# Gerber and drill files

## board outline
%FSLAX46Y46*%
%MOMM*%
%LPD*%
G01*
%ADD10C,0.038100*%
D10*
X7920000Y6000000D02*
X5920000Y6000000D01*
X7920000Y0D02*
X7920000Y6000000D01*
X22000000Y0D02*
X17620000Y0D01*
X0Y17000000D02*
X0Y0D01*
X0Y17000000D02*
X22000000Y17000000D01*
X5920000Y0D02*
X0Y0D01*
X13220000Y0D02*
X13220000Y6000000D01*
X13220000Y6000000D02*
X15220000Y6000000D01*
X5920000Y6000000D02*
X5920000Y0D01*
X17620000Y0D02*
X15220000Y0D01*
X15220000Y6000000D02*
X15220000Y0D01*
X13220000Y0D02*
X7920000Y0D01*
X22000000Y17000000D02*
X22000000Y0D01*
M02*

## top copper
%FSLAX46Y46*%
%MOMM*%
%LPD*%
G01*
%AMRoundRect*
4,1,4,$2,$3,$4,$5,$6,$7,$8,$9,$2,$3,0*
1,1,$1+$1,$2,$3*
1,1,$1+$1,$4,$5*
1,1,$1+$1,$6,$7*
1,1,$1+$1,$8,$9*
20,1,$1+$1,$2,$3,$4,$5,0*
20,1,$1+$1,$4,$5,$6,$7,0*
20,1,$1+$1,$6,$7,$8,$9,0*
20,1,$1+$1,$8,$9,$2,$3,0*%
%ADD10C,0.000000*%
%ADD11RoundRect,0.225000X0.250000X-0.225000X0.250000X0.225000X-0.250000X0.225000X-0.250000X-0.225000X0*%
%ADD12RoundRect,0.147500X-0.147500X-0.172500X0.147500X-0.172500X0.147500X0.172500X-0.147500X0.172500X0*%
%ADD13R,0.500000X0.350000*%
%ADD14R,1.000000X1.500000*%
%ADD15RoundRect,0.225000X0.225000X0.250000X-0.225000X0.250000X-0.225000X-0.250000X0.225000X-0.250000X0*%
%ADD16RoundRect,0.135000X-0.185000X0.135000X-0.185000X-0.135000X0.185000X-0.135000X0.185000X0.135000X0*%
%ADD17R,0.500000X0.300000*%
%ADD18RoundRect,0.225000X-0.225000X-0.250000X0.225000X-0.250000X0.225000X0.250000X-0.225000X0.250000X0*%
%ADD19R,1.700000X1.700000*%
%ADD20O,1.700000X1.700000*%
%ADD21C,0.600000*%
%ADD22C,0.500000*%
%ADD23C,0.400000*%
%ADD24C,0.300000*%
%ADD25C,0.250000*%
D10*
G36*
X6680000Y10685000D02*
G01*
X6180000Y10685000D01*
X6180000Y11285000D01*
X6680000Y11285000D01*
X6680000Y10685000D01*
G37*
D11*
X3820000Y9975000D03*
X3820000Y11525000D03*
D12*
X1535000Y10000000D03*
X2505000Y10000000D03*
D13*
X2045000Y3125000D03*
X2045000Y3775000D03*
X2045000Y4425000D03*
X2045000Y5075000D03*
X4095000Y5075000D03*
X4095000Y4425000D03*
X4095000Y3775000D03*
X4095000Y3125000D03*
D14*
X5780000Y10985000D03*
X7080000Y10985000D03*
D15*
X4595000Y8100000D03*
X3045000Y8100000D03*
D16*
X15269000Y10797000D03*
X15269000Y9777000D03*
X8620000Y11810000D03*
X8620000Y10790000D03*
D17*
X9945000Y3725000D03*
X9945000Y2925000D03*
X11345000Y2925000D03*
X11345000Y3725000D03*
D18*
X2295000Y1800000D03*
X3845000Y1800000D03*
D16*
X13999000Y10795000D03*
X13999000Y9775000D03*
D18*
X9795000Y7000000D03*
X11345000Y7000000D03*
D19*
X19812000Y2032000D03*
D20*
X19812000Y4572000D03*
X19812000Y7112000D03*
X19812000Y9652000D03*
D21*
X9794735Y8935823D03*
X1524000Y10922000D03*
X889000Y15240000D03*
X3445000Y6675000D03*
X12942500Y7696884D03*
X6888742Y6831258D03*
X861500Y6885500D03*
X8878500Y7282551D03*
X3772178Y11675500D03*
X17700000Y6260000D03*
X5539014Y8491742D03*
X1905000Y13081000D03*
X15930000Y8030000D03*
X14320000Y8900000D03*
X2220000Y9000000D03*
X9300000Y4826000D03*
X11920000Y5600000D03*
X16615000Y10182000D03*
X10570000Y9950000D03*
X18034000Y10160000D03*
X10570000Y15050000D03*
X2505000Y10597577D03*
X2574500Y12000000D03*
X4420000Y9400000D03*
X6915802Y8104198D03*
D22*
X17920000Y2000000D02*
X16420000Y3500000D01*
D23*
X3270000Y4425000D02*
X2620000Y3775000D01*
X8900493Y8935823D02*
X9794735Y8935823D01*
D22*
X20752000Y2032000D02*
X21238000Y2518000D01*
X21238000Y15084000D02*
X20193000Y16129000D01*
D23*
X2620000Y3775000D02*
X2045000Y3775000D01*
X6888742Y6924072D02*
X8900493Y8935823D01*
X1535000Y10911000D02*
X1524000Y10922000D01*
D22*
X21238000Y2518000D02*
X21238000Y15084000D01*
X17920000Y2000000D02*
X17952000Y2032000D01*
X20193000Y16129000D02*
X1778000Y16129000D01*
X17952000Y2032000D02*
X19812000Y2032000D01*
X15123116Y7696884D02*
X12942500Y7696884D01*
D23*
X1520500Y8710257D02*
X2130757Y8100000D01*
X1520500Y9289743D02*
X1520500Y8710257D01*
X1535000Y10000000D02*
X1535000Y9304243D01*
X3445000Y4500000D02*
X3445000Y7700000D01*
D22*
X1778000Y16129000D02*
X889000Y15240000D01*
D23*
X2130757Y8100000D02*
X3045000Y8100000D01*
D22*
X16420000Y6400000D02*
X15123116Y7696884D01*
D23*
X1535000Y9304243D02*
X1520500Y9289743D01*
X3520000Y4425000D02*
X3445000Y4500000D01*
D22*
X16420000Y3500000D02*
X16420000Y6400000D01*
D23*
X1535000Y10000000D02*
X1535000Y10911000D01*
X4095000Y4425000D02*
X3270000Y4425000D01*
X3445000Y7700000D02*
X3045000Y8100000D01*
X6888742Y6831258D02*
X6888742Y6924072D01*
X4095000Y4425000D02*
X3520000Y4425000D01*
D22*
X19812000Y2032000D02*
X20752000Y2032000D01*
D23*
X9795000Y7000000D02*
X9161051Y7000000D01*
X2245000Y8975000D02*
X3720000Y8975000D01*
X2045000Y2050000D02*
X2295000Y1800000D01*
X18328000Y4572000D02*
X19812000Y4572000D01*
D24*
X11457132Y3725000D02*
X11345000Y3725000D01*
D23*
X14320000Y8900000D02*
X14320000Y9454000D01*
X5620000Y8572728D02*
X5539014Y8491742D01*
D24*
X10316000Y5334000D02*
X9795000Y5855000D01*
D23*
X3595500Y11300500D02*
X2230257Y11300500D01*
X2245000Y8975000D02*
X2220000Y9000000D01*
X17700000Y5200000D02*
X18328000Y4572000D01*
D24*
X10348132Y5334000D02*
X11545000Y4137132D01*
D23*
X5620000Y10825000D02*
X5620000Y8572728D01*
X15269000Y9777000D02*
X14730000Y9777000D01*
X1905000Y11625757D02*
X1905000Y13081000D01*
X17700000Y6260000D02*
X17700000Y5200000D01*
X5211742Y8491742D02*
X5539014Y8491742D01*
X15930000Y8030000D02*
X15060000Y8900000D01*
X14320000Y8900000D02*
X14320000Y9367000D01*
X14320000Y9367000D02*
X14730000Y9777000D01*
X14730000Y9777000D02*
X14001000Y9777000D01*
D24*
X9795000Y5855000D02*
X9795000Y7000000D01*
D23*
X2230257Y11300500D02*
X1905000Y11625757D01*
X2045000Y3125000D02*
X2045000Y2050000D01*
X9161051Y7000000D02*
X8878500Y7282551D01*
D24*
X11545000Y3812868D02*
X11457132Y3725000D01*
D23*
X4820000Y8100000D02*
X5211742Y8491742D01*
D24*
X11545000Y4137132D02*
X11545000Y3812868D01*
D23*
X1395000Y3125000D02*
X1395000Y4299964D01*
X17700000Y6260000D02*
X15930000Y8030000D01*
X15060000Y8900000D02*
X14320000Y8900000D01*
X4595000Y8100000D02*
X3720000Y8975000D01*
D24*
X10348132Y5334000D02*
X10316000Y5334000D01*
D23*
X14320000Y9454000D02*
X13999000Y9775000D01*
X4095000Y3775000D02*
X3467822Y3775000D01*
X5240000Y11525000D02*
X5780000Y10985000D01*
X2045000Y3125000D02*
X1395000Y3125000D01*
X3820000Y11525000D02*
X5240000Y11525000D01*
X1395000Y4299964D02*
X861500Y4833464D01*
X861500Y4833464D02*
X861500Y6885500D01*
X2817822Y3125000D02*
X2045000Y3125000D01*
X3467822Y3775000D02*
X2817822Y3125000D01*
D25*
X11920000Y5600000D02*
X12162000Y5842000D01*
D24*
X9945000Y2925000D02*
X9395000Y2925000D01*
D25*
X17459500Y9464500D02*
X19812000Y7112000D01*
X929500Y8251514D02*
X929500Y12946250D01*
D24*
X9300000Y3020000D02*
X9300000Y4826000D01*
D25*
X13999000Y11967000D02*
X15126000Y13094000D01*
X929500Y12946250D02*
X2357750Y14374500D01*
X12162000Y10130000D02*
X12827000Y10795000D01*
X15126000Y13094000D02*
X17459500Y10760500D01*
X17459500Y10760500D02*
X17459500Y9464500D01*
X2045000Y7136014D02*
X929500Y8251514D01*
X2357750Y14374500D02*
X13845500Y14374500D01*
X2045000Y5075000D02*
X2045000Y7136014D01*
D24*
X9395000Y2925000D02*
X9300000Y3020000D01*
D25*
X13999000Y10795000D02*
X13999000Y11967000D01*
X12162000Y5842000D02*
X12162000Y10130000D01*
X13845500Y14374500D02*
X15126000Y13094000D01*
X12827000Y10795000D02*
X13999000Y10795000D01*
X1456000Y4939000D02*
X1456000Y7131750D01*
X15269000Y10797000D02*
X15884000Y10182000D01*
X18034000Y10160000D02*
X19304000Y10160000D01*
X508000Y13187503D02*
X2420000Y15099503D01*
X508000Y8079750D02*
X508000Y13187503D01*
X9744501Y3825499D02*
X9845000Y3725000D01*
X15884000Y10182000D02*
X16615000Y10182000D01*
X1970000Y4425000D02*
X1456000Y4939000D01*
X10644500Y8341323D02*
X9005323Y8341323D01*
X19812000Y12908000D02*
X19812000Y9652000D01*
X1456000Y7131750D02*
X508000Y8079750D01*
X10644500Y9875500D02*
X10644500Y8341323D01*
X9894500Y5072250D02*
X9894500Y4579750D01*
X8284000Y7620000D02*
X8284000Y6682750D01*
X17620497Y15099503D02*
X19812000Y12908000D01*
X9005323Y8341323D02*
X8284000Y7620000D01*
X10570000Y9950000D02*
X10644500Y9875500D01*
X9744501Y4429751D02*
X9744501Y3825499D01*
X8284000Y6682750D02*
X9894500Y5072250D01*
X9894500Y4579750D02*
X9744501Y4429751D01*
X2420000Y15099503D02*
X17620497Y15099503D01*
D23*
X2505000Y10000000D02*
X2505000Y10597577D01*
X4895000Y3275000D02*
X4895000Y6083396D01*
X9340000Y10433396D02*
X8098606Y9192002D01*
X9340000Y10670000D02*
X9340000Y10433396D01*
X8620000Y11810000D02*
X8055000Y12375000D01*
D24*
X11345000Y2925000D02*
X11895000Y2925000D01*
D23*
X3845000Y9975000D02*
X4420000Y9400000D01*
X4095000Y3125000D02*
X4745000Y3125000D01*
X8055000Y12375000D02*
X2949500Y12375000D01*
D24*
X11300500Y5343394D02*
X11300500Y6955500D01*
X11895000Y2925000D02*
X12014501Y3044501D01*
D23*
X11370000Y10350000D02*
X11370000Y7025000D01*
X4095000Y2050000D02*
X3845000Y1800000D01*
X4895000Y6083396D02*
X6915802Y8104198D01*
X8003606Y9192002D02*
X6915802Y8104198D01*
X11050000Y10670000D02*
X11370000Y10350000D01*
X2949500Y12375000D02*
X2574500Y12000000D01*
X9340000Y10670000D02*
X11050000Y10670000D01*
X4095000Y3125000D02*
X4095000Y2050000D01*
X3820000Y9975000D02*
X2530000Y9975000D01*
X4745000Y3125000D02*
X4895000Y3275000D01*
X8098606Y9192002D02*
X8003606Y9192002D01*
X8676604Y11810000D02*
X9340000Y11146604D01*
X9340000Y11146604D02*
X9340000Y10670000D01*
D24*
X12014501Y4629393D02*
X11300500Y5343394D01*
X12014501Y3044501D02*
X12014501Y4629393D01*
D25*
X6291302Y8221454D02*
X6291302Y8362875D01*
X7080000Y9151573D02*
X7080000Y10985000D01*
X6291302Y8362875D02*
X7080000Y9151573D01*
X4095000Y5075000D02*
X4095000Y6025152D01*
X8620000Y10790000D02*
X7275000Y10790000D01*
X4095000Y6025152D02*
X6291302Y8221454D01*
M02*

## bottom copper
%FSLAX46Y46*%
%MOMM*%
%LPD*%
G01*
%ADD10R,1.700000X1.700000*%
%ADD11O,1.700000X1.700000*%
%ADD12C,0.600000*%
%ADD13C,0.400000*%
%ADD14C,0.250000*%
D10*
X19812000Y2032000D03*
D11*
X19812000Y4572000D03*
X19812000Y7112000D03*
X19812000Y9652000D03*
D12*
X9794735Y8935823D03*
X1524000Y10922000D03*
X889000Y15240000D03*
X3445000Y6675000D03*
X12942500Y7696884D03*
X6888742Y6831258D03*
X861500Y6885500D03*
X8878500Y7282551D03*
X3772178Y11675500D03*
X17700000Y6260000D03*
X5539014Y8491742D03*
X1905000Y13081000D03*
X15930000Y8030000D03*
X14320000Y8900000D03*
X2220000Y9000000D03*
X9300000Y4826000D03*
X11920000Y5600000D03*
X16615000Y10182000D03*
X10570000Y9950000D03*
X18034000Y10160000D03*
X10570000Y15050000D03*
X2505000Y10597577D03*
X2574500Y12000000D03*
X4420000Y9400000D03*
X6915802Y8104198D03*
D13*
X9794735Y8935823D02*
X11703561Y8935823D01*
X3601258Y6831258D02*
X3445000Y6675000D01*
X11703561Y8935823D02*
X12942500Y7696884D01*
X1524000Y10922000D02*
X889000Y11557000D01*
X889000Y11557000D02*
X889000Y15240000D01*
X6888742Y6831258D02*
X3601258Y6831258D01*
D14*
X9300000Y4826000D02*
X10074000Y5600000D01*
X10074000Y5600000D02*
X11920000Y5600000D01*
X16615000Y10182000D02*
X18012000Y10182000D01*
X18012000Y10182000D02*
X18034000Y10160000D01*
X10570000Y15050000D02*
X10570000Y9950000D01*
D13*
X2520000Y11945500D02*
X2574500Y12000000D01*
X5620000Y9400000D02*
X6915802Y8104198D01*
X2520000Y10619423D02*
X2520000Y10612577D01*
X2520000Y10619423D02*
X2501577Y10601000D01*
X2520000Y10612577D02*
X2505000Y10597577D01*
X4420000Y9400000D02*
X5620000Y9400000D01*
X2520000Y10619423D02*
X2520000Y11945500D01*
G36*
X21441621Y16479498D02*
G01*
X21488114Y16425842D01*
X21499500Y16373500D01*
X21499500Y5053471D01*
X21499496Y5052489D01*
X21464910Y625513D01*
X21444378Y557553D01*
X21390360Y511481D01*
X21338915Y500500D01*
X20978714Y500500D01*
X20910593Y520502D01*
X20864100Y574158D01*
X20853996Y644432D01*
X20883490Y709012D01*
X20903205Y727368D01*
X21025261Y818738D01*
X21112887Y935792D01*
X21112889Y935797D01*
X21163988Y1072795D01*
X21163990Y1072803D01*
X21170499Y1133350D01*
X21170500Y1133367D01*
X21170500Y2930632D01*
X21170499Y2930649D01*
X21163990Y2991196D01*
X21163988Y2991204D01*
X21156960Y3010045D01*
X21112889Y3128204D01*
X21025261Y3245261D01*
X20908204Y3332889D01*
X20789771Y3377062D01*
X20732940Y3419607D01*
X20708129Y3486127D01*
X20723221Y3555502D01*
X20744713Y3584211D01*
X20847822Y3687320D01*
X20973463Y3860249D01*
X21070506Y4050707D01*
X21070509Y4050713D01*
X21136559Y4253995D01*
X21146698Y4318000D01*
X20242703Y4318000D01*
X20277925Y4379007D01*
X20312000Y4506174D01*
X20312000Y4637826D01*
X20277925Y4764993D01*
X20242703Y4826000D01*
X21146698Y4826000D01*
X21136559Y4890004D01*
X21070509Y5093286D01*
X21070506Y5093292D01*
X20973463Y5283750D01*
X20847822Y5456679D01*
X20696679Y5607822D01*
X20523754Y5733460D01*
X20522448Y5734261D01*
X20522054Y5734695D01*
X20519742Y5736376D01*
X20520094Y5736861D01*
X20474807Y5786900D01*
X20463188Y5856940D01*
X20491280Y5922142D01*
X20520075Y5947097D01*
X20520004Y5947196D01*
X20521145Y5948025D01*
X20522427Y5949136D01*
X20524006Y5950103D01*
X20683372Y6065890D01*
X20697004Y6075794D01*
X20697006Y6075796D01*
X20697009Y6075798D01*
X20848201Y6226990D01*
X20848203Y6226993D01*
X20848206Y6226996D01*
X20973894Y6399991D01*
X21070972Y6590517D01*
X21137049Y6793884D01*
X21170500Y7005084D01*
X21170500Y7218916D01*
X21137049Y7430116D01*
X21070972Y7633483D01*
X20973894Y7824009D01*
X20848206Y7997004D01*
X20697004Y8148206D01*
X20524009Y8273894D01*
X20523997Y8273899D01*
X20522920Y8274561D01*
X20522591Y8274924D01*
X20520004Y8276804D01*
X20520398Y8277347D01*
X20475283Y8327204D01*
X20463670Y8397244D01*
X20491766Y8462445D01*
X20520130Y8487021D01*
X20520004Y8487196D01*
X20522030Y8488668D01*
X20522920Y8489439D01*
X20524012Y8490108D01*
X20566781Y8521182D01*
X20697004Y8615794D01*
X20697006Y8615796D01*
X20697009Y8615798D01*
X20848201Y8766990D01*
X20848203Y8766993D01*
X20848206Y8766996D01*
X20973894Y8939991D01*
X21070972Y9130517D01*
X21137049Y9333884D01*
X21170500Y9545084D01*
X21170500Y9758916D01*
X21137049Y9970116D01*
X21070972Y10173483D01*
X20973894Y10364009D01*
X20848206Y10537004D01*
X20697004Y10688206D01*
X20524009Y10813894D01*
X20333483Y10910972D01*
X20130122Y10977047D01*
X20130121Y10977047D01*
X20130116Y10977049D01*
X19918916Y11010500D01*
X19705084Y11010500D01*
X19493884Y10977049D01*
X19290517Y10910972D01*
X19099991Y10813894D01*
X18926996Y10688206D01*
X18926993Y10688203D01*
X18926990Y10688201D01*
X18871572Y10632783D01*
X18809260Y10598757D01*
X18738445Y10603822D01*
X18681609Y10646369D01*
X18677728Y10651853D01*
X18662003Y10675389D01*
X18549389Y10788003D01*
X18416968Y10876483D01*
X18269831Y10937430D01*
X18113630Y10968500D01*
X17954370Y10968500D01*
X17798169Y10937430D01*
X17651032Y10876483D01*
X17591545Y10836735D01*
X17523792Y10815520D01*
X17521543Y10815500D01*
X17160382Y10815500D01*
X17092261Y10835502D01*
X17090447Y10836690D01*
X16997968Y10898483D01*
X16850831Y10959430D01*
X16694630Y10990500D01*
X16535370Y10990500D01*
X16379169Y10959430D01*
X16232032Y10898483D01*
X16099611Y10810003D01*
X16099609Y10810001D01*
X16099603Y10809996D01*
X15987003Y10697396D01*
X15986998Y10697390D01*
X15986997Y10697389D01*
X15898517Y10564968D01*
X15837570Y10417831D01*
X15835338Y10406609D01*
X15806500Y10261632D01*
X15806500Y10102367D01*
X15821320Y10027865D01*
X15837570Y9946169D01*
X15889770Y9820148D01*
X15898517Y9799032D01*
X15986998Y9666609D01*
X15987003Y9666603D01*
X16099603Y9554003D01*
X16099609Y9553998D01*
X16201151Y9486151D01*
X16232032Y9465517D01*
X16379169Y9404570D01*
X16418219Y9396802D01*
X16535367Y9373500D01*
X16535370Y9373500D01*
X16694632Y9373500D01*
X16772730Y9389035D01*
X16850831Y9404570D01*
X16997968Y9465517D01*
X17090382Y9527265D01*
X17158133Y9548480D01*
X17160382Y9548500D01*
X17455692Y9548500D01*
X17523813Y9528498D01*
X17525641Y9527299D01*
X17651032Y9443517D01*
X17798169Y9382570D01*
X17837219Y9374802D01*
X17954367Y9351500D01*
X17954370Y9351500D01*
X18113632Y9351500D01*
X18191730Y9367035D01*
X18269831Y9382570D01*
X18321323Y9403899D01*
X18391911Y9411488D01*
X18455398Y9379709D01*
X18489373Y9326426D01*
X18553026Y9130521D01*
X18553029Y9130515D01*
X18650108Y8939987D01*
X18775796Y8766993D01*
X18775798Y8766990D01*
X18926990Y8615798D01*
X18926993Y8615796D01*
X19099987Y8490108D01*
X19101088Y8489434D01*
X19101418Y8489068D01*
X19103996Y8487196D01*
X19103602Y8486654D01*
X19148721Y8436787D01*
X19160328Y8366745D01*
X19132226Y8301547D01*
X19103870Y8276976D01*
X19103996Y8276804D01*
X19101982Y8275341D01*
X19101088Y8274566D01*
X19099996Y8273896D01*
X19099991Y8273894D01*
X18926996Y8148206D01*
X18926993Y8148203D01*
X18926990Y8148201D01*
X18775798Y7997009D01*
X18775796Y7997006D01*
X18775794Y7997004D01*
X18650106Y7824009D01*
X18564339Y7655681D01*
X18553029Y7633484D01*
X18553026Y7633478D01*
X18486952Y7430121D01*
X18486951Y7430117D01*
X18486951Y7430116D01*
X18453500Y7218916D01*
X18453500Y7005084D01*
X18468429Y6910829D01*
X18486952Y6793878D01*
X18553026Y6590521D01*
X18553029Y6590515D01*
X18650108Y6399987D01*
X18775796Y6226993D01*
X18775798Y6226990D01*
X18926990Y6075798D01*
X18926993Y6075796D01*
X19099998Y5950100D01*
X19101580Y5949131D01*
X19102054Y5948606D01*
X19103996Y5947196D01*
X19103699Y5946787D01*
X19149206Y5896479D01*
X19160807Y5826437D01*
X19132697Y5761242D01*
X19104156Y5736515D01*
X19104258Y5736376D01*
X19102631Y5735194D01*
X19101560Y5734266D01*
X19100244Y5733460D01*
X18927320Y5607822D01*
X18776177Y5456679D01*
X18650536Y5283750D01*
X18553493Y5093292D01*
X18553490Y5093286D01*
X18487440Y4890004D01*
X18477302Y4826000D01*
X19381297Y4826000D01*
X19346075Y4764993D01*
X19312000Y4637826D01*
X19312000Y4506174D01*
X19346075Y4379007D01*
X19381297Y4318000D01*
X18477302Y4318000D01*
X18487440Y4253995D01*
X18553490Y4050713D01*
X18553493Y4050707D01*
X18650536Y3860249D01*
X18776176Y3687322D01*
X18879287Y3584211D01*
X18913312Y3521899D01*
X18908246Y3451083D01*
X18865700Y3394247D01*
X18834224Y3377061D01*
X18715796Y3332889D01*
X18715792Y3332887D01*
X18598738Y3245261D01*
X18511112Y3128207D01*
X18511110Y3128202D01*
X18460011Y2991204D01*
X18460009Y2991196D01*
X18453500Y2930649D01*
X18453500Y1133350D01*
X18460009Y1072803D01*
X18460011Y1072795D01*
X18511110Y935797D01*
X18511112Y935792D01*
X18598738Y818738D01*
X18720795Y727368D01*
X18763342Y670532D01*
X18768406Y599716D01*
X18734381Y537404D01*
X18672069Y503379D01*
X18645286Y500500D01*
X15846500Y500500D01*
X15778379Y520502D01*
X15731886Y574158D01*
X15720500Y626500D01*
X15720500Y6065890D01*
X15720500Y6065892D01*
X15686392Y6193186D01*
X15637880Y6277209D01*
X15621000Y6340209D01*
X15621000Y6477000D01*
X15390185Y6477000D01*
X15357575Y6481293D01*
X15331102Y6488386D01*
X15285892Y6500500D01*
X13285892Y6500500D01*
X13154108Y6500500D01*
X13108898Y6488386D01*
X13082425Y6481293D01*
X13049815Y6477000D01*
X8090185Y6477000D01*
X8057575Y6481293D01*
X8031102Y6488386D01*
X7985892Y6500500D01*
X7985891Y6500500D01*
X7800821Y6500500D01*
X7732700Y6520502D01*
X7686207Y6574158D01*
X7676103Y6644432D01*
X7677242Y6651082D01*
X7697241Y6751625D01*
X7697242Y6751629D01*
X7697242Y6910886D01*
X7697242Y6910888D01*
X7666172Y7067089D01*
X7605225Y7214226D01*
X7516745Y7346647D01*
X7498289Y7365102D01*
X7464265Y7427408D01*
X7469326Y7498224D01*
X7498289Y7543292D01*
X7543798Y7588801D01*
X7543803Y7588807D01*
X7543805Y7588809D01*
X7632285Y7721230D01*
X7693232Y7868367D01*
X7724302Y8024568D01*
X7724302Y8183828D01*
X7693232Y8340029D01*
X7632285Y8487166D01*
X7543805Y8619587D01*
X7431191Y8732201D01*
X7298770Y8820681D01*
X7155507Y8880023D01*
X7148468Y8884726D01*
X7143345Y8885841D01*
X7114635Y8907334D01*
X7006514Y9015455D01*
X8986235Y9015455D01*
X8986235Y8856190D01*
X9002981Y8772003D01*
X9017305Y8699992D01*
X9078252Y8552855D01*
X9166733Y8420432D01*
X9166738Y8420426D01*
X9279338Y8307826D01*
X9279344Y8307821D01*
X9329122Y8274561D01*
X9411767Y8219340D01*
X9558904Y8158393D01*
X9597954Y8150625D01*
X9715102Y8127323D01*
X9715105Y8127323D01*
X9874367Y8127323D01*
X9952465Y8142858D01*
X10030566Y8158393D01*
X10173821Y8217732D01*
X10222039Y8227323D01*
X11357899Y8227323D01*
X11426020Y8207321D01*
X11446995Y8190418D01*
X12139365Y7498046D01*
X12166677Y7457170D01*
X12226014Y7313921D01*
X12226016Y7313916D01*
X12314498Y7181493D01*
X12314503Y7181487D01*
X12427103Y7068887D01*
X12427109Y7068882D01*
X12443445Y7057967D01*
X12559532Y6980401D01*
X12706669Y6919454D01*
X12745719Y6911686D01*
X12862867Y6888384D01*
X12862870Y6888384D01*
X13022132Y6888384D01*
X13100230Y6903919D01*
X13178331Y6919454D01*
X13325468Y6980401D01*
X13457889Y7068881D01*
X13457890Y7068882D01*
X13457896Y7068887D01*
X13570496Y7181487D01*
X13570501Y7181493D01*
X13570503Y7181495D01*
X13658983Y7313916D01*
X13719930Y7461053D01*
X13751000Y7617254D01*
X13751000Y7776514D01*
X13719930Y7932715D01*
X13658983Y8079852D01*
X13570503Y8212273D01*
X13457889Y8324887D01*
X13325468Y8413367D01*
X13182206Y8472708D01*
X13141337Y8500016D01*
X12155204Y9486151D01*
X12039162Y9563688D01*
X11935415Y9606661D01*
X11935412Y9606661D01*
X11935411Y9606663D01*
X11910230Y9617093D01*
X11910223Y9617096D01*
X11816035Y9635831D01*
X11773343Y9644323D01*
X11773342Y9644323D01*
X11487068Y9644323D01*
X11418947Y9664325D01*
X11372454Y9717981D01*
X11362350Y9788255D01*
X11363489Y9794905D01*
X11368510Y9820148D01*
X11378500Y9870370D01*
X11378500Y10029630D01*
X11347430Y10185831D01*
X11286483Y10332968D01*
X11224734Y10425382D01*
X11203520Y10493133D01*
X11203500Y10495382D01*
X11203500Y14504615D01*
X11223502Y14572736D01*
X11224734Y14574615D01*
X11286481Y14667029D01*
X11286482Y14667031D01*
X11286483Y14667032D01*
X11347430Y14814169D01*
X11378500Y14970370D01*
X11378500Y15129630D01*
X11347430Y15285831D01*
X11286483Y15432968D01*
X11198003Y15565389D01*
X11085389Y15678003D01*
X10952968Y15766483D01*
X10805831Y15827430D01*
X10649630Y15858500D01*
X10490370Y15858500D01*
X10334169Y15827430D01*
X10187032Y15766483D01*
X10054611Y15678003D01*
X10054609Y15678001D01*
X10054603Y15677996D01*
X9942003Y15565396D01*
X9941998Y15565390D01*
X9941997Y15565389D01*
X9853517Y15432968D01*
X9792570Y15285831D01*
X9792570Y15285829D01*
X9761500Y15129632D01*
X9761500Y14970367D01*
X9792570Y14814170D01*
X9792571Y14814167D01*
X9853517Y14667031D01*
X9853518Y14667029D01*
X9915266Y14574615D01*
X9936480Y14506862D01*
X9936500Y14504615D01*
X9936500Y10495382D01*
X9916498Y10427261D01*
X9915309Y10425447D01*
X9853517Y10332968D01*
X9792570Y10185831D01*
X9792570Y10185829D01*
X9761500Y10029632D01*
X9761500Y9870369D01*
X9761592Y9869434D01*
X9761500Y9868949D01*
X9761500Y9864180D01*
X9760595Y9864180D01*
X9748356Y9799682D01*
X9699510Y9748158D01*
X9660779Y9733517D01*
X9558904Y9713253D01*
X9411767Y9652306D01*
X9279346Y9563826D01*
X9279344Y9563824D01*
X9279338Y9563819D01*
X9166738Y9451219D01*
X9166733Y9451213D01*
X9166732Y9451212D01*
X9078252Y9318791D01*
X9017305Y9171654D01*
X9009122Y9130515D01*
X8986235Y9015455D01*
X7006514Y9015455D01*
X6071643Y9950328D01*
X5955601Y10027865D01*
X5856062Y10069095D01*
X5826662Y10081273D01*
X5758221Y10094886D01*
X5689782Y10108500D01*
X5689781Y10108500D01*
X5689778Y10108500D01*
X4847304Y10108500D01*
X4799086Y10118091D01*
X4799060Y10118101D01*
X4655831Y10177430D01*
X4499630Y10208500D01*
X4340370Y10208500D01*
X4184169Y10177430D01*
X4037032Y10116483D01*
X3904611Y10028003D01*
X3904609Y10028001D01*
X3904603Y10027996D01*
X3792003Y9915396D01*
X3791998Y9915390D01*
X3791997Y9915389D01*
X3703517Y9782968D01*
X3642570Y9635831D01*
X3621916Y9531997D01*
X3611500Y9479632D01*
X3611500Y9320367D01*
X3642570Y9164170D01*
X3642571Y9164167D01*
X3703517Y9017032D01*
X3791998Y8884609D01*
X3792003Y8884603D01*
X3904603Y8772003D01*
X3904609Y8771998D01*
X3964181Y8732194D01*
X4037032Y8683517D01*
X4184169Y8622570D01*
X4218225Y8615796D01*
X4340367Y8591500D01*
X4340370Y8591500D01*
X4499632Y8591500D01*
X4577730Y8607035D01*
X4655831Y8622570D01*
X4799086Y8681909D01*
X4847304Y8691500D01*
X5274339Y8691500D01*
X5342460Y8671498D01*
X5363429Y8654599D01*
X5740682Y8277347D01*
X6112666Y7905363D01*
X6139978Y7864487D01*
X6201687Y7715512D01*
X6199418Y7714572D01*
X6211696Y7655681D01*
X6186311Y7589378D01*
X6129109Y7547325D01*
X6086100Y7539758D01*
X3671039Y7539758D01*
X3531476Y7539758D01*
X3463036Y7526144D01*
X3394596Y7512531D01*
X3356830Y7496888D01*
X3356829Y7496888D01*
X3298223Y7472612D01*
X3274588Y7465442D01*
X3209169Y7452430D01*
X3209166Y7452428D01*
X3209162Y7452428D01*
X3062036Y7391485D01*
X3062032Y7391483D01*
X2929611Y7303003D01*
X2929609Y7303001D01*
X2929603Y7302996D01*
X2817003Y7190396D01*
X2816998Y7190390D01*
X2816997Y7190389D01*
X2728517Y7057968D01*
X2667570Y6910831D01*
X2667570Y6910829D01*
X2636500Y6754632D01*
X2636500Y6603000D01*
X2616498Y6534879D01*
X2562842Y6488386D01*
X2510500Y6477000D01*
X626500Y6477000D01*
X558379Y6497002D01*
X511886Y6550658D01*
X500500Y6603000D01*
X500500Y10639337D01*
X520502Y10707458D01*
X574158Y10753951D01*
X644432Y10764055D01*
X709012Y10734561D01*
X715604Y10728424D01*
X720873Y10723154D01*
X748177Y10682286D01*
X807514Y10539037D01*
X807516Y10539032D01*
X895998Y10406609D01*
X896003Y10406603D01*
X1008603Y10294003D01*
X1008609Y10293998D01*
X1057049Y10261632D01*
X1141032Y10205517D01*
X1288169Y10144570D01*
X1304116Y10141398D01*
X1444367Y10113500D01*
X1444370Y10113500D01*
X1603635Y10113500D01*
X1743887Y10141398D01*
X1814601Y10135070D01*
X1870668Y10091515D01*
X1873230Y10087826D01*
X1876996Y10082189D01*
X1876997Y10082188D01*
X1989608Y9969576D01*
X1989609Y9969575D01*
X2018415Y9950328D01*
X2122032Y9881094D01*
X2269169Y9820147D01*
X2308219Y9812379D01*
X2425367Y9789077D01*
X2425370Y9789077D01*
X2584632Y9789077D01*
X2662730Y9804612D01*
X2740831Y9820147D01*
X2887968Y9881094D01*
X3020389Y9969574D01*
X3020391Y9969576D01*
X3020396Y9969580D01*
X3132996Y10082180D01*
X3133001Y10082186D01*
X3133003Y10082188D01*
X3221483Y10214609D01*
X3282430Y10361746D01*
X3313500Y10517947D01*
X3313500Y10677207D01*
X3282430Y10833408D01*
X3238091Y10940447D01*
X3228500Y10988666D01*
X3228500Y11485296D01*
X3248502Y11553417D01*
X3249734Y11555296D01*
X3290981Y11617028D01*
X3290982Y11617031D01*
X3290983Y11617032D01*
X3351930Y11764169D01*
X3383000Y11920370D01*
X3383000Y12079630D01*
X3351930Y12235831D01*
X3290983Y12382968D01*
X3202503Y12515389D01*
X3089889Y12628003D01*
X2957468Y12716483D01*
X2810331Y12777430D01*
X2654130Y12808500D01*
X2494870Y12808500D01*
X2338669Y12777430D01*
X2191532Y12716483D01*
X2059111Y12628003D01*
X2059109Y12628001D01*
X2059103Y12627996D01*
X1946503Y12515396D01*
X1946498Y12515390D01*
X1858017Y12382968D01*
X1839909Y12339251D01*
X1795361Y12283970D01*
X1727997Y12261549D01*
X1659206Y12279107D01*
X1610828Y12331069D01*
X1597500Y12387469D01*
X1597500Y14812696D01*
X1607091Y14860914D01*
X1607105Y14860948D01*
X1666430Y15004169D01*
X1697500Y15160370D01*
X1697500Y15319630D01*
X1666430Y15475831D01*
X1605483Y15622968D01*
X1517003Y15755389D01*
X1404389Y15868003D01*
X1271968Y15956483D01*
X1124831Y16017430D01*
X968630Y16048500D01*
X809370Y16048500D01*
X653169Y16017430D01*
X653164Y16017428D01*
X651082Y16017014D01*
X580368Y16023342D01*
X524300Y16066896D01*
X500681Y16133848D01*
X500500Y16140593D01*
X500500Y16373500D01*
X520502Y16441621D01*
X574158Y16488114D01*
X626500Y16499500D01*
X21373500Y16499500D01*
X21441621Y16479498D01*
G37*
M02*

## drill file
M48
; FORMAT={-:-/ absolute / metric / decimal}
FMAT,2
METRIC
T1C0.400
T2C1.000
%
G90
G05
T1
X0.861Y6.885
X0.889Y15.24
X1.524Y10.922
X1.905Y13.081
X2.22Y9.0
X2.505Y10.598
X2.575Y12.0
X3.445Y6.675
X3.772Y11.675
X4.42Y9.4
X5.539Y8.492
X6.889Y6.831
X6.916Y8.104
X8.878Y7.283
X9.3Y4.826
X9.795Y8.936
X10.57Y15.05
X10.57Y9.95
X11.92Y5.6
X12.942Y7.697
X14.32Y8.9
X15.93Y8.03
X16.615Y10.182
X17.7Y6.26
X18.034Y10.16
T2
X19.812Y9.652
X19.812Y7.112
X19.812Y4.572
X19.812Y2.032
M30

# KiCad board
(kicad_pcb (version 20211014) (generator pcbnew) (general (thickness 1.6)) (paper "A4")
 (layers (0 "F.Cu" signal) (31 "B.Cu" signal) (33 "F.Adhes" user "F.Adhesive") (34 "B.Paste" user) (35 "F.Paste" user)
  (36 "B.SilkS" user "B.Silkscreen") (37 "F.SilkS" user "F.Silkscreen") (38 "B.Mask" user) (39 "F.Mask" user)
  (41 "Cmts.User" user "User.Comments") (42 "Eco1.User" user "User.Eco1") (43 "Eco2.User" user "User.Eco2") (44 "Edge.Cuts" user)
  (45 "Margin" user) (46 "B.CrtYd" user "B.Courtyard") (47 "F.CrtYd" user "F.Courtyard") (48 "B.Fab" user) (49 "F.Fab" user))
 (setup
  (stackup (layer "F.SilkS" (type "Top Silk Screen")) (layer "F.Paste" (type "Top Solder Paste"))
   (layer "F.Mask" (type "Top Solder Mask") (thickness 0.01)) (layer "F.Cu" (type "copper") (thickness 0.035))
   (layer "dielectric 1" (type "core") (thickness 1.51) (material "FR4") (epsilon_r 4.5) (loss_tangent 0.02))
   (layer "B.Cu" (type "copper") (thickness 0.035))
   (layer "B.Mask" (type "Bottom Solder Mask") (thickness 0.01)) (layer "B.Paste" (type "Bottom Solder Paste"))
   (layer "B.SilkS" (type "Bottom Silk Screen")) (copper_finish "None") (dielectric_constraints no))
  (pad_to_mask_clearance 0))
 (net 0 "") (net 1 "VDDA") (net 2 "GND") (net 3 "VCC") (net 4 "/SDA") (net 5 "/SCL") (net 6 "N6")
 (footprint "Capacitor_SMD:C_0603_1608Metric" (layer "F.Cu") (at 3.82 -10.75 90)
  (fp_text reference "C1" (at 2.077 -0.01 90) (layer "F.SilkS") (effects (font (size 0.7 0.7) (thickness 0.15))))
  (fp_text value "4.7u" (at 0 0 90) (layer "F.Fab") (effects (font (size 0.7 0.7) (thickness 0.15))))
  (pad "1" smd roundrect (at -0.775 0 90) (size 0.9 0.95) (layers "F.Cu" "F.Paste" "F.Mask") (roundrect_rratio 0.25) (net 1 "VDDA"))
  (pad "2" smd roundrect (at 0.775 0 90) (size 0.9 0.95) (layers "F.Cu" "F.Paste" "F.Mask") (roundrect_rratio 0.25) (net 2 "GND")))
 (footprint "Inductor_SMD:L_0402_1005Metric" (layer "F.Cu") (at 2.02 -10)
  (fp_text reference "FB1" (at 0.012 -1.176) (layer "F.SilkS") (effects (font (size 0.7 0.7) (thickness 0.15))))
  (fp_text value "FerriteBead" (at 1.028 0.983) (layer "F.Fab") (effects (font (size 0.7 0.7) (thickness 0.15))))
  (pad "1" smd roundrect (at -0.485 0) (size 0.59 0.64) (layers "F.Cu" "F.Paste" "F.Mask") (roundrect_rratio 0.25) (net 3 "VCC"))
  (pad "2" smd roundrect (at 0.485 0) (size 0.59 0.64) (layers "F.Cu" "F.Paste" "F.Mask") (roundrect_rratio 0.25) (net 1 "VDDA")))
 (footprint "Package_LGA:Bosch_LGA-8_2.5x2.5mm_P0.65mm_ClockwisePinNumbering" (layer "F.Cu") (at 3.07 -4.1 90)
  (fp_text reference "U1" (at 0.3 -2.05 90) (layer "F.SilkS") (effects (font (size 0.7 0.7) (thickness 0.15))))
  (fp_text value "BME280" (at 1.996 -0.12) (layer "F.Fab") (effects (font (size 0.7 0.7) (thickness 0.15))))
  (pad "1" smd rect (at -0.975 -1.025 180) (size 0.5 0.35) (layers "F.Cu" "F.Paste" "F.Mask") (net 2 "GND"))
  (pad "2" smd rect (at -0.325 -1.025 180) (size 0.5 0.35) (layers "F.Cu" "F.Paste" "F.Mask") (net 3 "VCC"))
  (pad "3" smd rect (at 0.325 -1.025 180) (size 0.5 0.35) (layers "F.Cu" "F.Paste" "F.Mask") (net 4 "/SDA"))
  (pad "4" smd rect (at 0.975 -1.025 180) (size 0.5 0.35) (layers "F.Cu" "F.Paste" "F.Mask") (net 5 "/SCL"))
  (pad "5" smd rect (at 0.975 1.025 180) (size 0.5 0.35) (layers "F.Cu" "F.Paste" "F.Mask") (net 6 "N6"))
  (pad "6" smd rect (at 0.325 1.025 180) (size 0.5 0.35) (layers "F.Cu" "F.Paste" "F.Mask") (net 3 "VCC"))
  (pad "7" smd rect (at -0.325 1.025 180) (size 0.5 0.35) (layers "F.Cu" "F.Paste" "F.Mask") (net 2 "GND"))
  (pad "8" smd rect (at -0.975 1.025 180) (size 0.5 0.35) (layers "F.Cu" "F.Paste" "F.Mask") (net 1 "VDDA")))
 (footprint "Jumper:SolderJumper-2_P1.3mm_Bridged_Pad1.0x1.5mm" (layer "F.Cu") (at 6.43 -10.985)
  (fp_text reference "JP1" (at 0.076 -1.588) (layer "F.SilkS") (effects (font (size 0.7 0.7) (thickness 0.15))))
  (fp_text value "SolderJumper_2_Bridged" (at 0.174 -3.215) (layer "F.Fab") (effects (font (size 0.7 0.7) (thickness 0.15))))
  (fp_poly (pts (xy -0.25 -0.3) (xy 0.25 -0.3) (xy 0.25 0.3) (xy -0.25 0.3)) (layer "F.Cu") (width 0) (fill solid))
  (pad "1" smd rect (at -0.65 0) (size 1 1.5) (layers "F.Cu" "F.Mask") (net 2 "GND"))
  (pad "2" smd rect (at 0.65 0) (size 1 1.5) (layers "F.Cu" "F.Mask") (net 6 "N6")))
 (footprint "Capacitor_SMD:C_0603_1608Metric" (layer "F.Cu") (at 3.82 -8.1 180)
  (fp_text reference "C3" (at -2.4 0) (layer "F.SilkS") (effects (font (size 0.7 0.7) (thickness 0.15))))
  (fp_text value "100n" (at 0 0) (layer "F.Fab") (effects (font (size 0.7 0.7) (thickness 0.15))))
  (pad "1" smd roundrect (at -0.775 0 180) (size 0.9 0.95) (layers "F.Cu" "F.Paste" "F.Mask") (roundrect_rratio 0.25) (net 2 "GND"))
  (pad "2" smd roundrect (at 0.775 0 180) (size 0.9 0.95) (layers "F.Cu" "F.Paste" "F.Mask") (roundrect_rratio 0.25) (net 3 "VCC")))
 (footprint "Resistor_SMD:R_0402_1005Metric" (layer "F.Cu") (at 15.269 -10.287 -90)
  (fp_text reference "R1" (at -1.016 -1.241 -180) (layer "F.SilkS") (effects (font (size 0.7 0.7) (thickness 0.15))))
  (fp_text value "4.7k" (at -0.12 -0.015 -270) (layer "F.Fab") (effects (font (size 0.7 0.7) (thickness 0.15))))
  (pad "1" smd roundrect (at -0.51 0 270) (size 0.54 0.64) (layers "F.Cu" "F.Paste" "F.Mask") (roundrect_rratio 0.25) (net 4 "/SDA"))
  (pad "2" smd roundrect (at 0.51 0 270) (size 0.54 0.64) (layers "F.Cu" "F.Paste" "F.Mask") (roundrect_rratio 0.25) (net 2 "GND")))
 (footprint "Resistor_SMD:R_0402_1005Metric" (layer "F.Cu") (at 8.62 -11.3 -90)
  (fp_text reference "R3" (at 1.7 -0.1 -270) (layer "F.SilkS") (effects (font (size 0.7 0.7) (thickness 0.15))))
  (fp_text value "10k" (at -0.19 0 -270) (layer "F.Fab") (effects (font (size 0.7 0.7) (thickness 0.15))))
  (pad "1" smd roundrect (at -0.51 0 270) (size 0.54 0.64) (layers "F.Cu" "F.Paste" "F.Mask") (roundrect_rratio 0.25) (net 1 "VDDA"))
  (pad "2" smd roundrect (at 0.51 0 270) (size 0.54 0.64) (layers "F.Cu" "F.Paste" "F.Mask") (roundrect_rratio 0.25) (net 6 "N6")))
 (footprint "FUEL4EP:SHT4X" (layer "F.Cu") (at 10.645 -3.325)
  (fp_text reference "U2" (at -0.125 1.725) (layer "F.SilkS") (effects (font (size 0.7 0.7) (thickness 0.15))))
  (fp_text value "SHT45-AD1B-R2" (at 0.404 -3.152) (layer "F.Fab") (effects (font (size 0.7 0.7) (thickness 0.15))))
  (pad "1" smd rect (at -0.7 -0.4) (size 0.5 0.3) (layers "F.Cu" "F.Paste" "F.Mask") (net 4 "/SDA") (solder_mask_margin 0.102))
  (pad "2" smd rect (at -0.7 0.4) (size 0.5 0.3) (layers "F.Cu" "F.Paste" "F.Mask") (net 5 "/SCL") (solder_mask_margin 0.102))
  (pad "3" smd rect (at 0.7 0.4) (size 0.5 0.3) (layers "F.Cu" "F.Paste" "F.Mask") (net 1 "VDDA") (solder_mask_margin 0.102))
  (pad "4" smd rect (at 0.7 -0.4) (size 0.5 0.3) (layers "F.Cu" "F.Paste" "F.Mask") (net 2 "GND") (solder_mask_margin 0.102)))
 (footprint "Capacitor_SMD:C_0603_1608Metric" (layer "F.Cu") (at 3.07 -1.8)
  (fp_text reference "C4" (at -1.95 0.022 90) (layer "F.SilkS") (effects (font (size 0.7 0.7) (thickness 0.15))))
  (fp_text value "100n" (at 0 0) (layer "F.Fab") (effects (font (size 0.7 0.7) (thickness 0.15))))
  (pad "1" smd roundrect (at -0.775 0) (size 0.9 0.95) (layers "F.Cu" "F.Paste" "F.Mask") (roundrect_rratio 0.25) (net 2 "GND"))
  (pad "2" smd roundrect (at 0.775 0) (size 0.9 0.95) (layers "F.Cu" "F.Paste" "F.Mask") (roundrect_rratio 0.25) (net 1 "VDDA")))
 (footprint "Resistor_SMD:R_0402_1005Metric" (layer "F.Cu") (at 13.999 -10.285 -90)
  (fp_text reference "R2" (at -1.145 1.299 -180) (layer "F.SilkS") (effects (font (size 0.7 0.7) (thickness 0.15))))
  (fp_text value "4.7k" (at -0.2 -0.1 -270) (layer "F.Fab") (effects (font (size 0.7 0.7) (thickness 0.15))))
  (pad "1" smd roundrect (at -0.51 0 270) (size 0.54 0.64) (layers "F.Cu" "F.Paste" "F.Mask") (roundrect_rratio 0.25) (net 5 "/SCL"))
  (pad "2" smd roundrect (at 0.51 0 270) (size 0.54 0.64) (layers "F.Cu" "F.Paste" "F.Mask") (roundrect_rratio 0.25) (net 2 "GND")))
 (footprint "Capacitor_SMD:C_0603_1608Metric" (layer "F.Cu") (at 10.57 -7)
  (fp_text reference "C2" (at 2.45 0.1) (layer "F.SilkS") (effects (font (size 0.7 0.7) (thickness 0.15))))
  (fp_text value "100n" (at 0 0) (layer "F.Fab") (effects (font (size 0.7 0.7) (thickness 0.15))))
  (pad "1" smd roundrect (at -0.775 0) (size 0.9 0.95) (layers "F.Cu" "F.Paste" "F.Mask") (roundrect_rratio 0.25) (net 2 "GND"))
  (pad "2" smd roundrect (at 0.775 0) (size 0.9 0.95) (layers "F.Cu" "F.Paste" "F.Mask") (roundrect_rratio 0.25) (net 1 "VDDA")))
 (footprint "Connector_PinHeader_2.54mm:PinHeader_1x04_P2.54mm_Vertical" (layer "B.Cu") (at 19.812 -2.032)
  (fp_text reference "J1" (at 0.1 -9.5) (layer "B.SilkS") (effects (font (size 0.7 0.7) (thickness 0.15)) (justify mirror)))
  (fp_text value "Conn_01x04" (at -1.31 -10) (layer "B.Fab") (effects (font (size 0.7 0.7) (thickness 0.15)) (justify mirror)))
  (pad "1" thru_hole rect (at 0 0) (size 1.7 1.7) (drill 1) (layers *.Cu *.Mask) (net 3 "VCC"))
  (pad "2" thru_hole oval (at 0 -2.54) (size 1.7 1.7) (drill 1) (layers *.Cu *.Mask) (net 2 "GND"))
  (pad "3" thru_hole oval (at 0 -5.08) (size 1.7 1.7) (drill 1) (layers *.Cu *.Mask) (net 5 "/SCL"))
  (pad "4" thru_hole oval (at 0 -7.62) (size 1.7 1.7) (drill 1) (layers *.Cu *.Mask) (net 4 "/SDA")))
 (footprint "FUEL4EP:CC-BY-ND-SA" (layer "B.Cu") (at 11.176 -14.351 180)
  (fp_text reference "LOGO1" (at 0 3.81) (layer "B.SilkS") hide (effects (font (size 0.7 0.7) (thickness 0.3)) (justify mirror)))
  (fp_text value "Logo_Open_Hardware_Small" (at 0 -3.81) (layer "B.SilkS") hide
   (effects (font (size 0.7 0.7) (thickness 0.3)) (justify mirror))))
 (gr_line (start 7.92 -6) (end 5.92 -6) (layer "Edge.Cuts") (width 0.0381))
 (gr_line (start 7.92 0) (end 7.92 -6) (layer "Edge.Cuts") (width 0.0381))
 (gr_line (start 22 0) (end 17.62 0) (layer "Edge.Cuts") (width 0.0381))
 (gr_line (start 0 -17) (end 0 0) (layer "Edge.Cuts") (width 0.0381))
 (gr_line (start 0 -17) (end 22 -17) (layer "Edge.Cuts") (width 0.0381))
 (gr_line (start 5.92 0) (end 0 0) (layer "Edge.Cuts") (width 0.0381))
 (gr_line (start 13.22 0) (end 13.22 -6) (layer "Edge.Cuts") (width 0.0381))
 (gr_line (start 13.22 -6) (end 15.22 -6) (layer "Edge.Cuts") (width 0.0381))
 (gr_line (start 5.92 -6) (end 5.92 0) (layer "Edge.Cuts") (width 0.0381))
 (gr_line (start 17.62 0) (end 15.22 0) (layer "Edge.Cuts") (width 0.0381))
 (gr_line (start 15.22 -6) (end 15.22 0) (layer "Edge.Cuts") (width 0.0381))
 (gr_line (start 13.22 0) (end 7.92 0) (layer "Edge.Cuts") (width 0.0381))
 (gr_line (start 22 -17) (end 22 0) (layer "Edge.Cuts") (width 0.0381))
 (segment (start 17.92 -2) (end 16.42 -3.5) (width 0.5) (layer "F.Cu") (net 3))
 (segment (start 3.27 -4.425) (end 2.62 -3.775) (width 0.4) (layer "F.Cu") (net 3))
 (segment (start 8.900493 -8.935823) (end 9.794735 -8.935823) (width 0.4) (layer "F.Cu") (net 3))
 (segment (start 20.752 -2.032) (end 21.238 -2.518) (width 0.5) (layer "F.Cu") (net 3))
 (segment (start 21.238 -15.084) (end 20.193 -16.129) (width 0.5) (layer "F.Cu") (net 3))
 (segment (start 2.62 -3.775) (end 2.045 -3.775) (width 0.4) (layer "F.Cu") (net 3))
 (segment (start 6.888742 -6.924072) (end 8.900493 -8.935823) (width 0.4) (layer "F.Cu") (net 3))
 (segment (start 1.535 -10.911) (end 1.524 -10.922) (width 0.4) (layer "F.Cu") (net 3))
 (segment (start 21.238 -2.518) (end 21.238 -15.084) (width 0.5) (layer "F.Cu") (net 3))
 (segment (start 17.92 -2) (end 17.952 -2.032) (width 0.5) (layer "F.Cu") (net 3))
 (segment (start 20.193 -16.129) (end 1.778 -16.129) (width 0.5) (layer "F.Cu") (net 3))
 (segment (start 17.952 -2.032) (end 19.812 -2.032) (width 0.5) (layer "F.Cu") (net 3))
 (segment (start 15.123116 -7.696884) (end 12.9425 -7.696884) (width 0.5) (layer "F.Cu") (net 3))
 (segment (start 1.5205 -8.710257) (end 2.130757 -8.1) (width 0.4) (layer "F.Cu") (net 3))
 (segment (start 1.5205 -9.289743) (end 1.5205 -8.710257) (width 0.4) (layer "F.Cu") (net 3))
 (segment (start 1.535 -10) (end 1.535 -9.304243) (width 0.4) (layer "F.Cu") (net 3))
 (segment (start 3.445 -4.5) (end 3.445 -7.7) (width 0.4) (layer "F.Cu") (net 3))
 (segment (start 1.778 -16.129) (end 0.889 -15.24) (width 0.5) (layer "F.Cu") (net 3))
 (segment (start 2.130757 -8.1) (end 3.045 -8.1) (width 0.4) (layer "F.Cu") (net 3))
 (segment (start 16.42 -6.4) (end 15.123116 -7.696884) (width 0.5) (layer "F.Cu") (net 3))
 (segment (start 1.535 -9.304243) (end 1.5205 -9.289743) (width 0.4) (layer "F.Cu") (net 3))
 (segment (start 3.52 -4.425) (end 3.445 -4.5) (width 0.4) (layer "F.Cu") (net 3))
 (segment (start 16.42 -3.5) (end 16.42 -6.4) (width 0.5) (layer "F.Cu") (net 3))
 (segment (start 1.535 -10) (end 1.535 -10.911) (width 0.4) (layer "F.Cu") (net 3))
 (segment (start 4.095 -4.425) (end 3.27 -4.425) (width 0.4) (layer "F.Cu") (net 3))
 (segment (start 3.445 -7.7) (end 3.045 -8.1) (width 0.4) (layer "F.Cu") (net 3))
 (segment (start 6.888742 -6.831258) (end 6.888742 -6.924072) (width 0.4) (layer "F.Cu") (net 3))
 (segment (start 4.095 -4.425) (end 3.52 -4.425) (width 0.4) (layer "F.Cu") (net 3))
 (segment (start 19.812 -2.032) (end 20.752 -2.032) (width 0.5) (layer "F.Cu") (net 3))
 (via (at 9.794735 -8.935823) (size 0.6) (drill 0.4) (layers "F.Cu" "B.Cu") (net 3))
 (via (at 1.524 -10.922) (size 0.6) (drill 0.4) (layers "F.Cu" "B.Cu") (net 3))
 (via (at 0.889 -15.24) (size 0.6) (drill 0.4) (layers "F.Cu" "B.Cu") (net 3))
 (via (at 3.445 -6.675) (size 0.6) (drill 0.4) (layers "F.Cu" "B.Cu") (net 3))
 (via (at 12.9425 -7.696884) (size 0.6) (drill 0.4) (layers "F.Cu" "B.Cu") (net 3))
 (via (at 6.888742 -6.831258) (size 0.6) (drill 0.4) (layers "F.Cu" "B.Cu") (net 3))
 (segment (start 9.794735 -8.935823) (end 11.703561 -8.935823) (width 0.4) (layer "B.Cu") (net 3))
 (segment (start 3.601258 -6.831258) (end 3.445 -6.675) (width 0.4) (layer "B.Cu") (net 3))
 (segment (start 11.703561 -8.935823) (end 12.9425 -7.696884) (width 0.4) (layer "B.Cu") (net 3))
 (segment (start 1.524 -10.922) (end 0.889 -11.557) (width 0.4) (layer "B.Cu") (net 3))
 (segment (start 0.889 -11.557) (end 0.889 -15.24) (width 0.4) (layer "B.Cu") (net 3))
 (segment (start 6.888742 -6.831258) (end 3.601258 -6.831258) (width 0.4) (layer "B.Cu") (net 3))
 (segment (start 9.795 -7) (end 9.161051 -7) (width 0.4) (layer "F.Cu") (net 2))
 (segment (start 2.245 -8.975) (end 3.72 -8.975) (width 0.4) (layer "F.Cu") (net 2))
 (segment (start 2.045 -2.05) (end 2.295 -1.8) (width 0.4) (layer "F.Cu") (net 2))
 (segment (start 18.328 -4.572) (end 19.812 -4.572) (width 0.4) (layer "F.Cu") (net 2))
 (segment (start 11.457132 -3.725) (end 11.345 -3.725) (width 0.3) (layer "F.Cu") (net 2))
 (segment (start 14.32 -8.9) (end 14.32 -9.454) (width 0.4) (layer "F.Cu") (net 2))
 (segment (start 5.62 -8.572728) (end 5.539014 -8.491742) (width 0.4) (layer "F.Cu") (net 2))
 (segment (start 10.316 -5.334) (end 9.795 -5.855) (width 0.3) (layer "F.Cu") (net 2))
 (segment (start 3.5955 -11.3005) (end 2.230257 -11.3005) (width 0.4) (layer "F.Cu") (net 2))
 (segment (start 2.245 -8.975) (end 2.22 -9) (width 0.4) (layer "F.Cu") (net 2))
 (segment (start 17.7 -5.2) (end 18.328 -4.572) (width 0.4) (layer "F.Cu") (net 2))
 (segment (start 10.348132 -5.334) (end 11.545 -4.137132) (width 0.3) (layer "F.Cu") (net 2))
 (segment (start 5.62 -10.825) (end 5.62 -8.572728) (width 0.4) (layer "F.Cu") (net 2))
 (segment (start 15.269 -9.777) (end 14.73 -9.777) (width 0.4) (layer "F.Cu") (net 2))
 (segment (start 1.905 -11.625757) (end 1.905 -13.081) (width 0.4) (layer "F.Cu") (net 2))
 (segment (start 17.7 -6.26) (end 17.7 -5.2) (width 0.4) (layer "F.Cu") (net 2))
 (segment (start 5.211742 -8.491742) (end 5.539014 -8.491742) (width 0.4) (layer "F.Cu") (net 2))
 (segment (start 15.93 -8.03) (end 15.06 -8.9) (width 0.4) (layer "F.Cu") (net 2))
 (segment (start 14.32 -8.9) (end 14.32 -9.367) (width 0.4) (layer "F.Cu") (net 2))
 (segment (start 14.32 -9.367) (end 14.73 -9.777) (width 0.4) (layer "F.Cu") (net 2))
 (segment (start 14.73 -9.777) (end 14.001 -9.777) (width 0.4) (layer "F.Cu") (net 2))
 (segment (start 9.795 -5.855) (end 9.795 -7) (width 0.3) (layer "F.Cu") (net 2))
 (segment (start 2.230257 -11.3005) (end 1.905 -11.625757) (width 0.4) (layer "F.Cu") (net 2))
 (segment (start 2.045 -3.125) (end 2.045 -2.05) (width 0.4) (layer "F.Cu") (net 2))
 (segment (start 9.161051 -7) (end 8.8785 -7.282551) (width 0.4) (layer "F.Cu") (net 2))
 (segment (start 11.545 -3.812868) (end 11.457132 -3.725) (width 0.3) (layer "F.Cu") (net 2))
 (segment (start 4.82 -8.1) (end 5.211742 -8.491742) (width 0.4) (layer "F.Cu") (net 2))
 (segment (start 11.545 -4.137132) (end 11.545 -3.812868) (width 0.3) (layer "F.Cu") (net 2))
 (segment (start 1.395 -3.125) (end 1.395 -4.299964) (width 0.4) (layer "F.Cu") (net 2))
 (segment (start 17.7 -6.26) (end 15.93 -8.03) (width 0.4) (layer "F.Cu") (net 2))
 (segment (start 15.06 -8.9) (end 14.32 -8.9) (width 0.4) (layer "F.Cu") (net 2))
 (segment (start 4.595 -8.1) (end 3.72 -8.975) (width 0.4) (layer "F.Cu") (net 2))
 (segment (start 10.348132 -5.334) (end 10.316 -5.334) (width 0.3) (layer "F.Cu") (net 2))
 (segment (start 14.32 -9.454) (end 13.999 -9.775) (width 0.4) (layer "F.Cu") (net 2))
 (segment (start 4.095 -3.775) (end 3.467822 -3.775) (width 0.4) (layer "F.Cu") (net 2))
 (segment (start 5.24 -11.525) (end 5.78 -10.985) (width 0.4) (layer "F.Cu") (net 2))
 (segment (start 2.045 -3.125) (end 1.395 -3.125) (width 0.4) (layer "F.Cu") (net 2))
 (segment (start 3.82 -11.525) (end 5.24 -11.525) (width 0.4) (layer "F.Cu") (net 2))
 (segment (start 1.395 -4.299964) (end 0.8615 -4.833464) (width 0.4) (layer "F.Cu") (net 2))
 (segment (start 0.8615 -4.833464) (end 0.8615 -6.8855) (width 0.4) (layer "F.Cu") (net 2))
 (segment (start 2.817822 -3.125) (end 2.045 -3.125) (width 0.4) (layer "F.Cu") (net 2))
 (segment (start 3.467822 -3.775) (end 2.817822 -3.125) (width 0.4) (layer "F.Cu") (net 2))
 (via (at 0.8615 -6.8855) (size 0.6) (drill 0.4) (layers "F.Cu" "B.Cu") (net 2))
 (via (at 8.8785 -7.282551) (size 0.6) (drill 0.4) (layers "F.Cu" "B.Cu") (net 2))
 (via (at 3.772178 -11.6755) (size 0.6) (drill 0.4) (layers "F.Cu" "B.Cu") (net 2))
 (via (at 17.7 -6.26) (size 0.6) (drill 0.4) (layers "F.Cu" "B.Cu") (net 2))
 (via (at 5.539014 -8.491742) (size 0.6) (drill 0.4) (layers "F.Cu" "B.Cu") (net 2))
 (via (at 1.905 -13.081) (size 0.6) (drill 0.4) (layers "F.Cu" "B.Cu") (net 2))
 (via (at 15.93 -8.03) (size 0.6) (drill 0.4) (layers "F.Cu" "B.Cu") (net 2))
 (via (at 14.32 -8.9) (size 0.6) (drill 0.4) (layers "F.Cu" "B.Cu") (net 2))
 (via (at 2.22 -9) (size 0.6) (drill 0.4) (layers "F.Cu" "B.Cu") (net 2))
 (segment (start 11.92 -5.6) (end 12.162 -5.842) (width 0.25) (layer "F.Cu") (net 5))
 (segment (start 9.945 -2.925) (end 9.395 -2.925) (width 0.3) (layer "F.Cu") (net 5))
 (segment (start 17.4595 -9.4645) (end 19.812 -7.112) (width 0.25) (layer "F.Cu") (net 5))
 (segment (start 0.9295 -8.251514) (end 0.9295 -12.94625) (width 0.25) (layer "F.Cu") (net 5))
 (segment (start 9.3 -3.02) (end 9.3 -4.826) (width 0.3) (layer "F.Cu") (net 5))
 (segment (start 13.999 -11.967) (end 15.126 -13.094) (width 0.25) (layer "F.Cu") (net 5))
 (segment (start 0.9295 -12.94625) (end 2.35775 -14.3745) (width 0.25) (layer "F.Cu") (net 5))
 (segment (start 12.162 -10.13) (end 12.827 -10.795) (width 0.25) (layer "F.Cu") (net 5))
 (segment (start 15.126 -13.094) (end 17.4595 -10.7605) (width 0.25) (layer "F.Cu") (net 5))
 (segment (start 17.4595 -10.7605) (end 17.4595 -9.4645) (width 0.25) (layer "F.Cu") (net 5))
 (segment (start 2.045 -7.136014) (end 0.9295 -8.251514) (width 0.25) (layer "F.Cu") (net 5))
 (segment (start 2.35775 -14.3745) (end 13.8455 -14.3745) (width 0.25) (layer "F.Cu") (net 5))
 (segment (start 2.045 -5.075) (end 2.045 -7.136014) (width 0.25) (layer "F.Cu") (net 5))
 (segment (start 9.395 -2.925) (end 9.3 -3.02) (width 0.3) (layer "F.Cu") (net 5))
 (segment (start 13.999 -10.795) (end 13.999 -11.967) (width 0.25) (layer "F.Cu") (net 5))
 (segment (start 12.162 -5.842) (end 12.162 -10.13) (width 0.25) (layer "F.Cu") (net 5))
 (segment (start 13.8455 -14.3745) (end 15.126 -13.094) (width 0.25) (layer "F.Cu") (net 5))
 (segment (start 12.827 -10.795) (end 13.999 -10.795) (width 0.25) (layer "F.Cu") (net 5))
 (via (at 9.3 -4.826) (size 0.6) (drill 0.4) (layers "F.Cu" "B.Cu") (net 5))
 (via (at 11.92 -5.6) (size 0.6) (drill 0.4) (layers "F.Cu" "B.Cu") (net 5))
 (segment (start 9.3 -4.826) (end 10.074 -5.6) (width 0.25) (layer "B.Cu") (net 5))
 (segment (start 10.074 -5.6) (end 11.92 -5.6) (width 0.25) (layer "B.Cu") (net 5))
 (segment (start 1.456 -4.939) (end 1.456 -7.13175) (width 0.25) (layer "F.Cu") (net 4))
 (segment (start 15.269 -10.797) (end 15.884 -10.182) (width 0.25) (layer "F.Cu") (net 4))
 (segment (start 18.034 -10.16) (end 19.304 -10.16) (width 0.25) (layer "F.Cu") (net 4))
 (segment (start 0.508 -13.187503) (end 2.42 -15.099503) (width 0.25) (layer "F.Cu") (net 4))
 (segment (start 0.508 -8.07975) (end 0.508 -13.187503) (width 0.25) (layer "F.Cu") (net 4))
 (segment (start 9.744501 -3.825499) (end 9.845 -3.725) (width 0.25) (layer "F.Cu") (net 4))
 (segment (start 15.884 -10.182) (end 16.615 -10.182) (width 0.25) (layer "F.Cu") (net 4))
 (segment (start 1.97 -4.425) (end 1.456 -4.939) (width 0.25) (layer "F.Cu") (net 4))
 (segment (start 10.6445 -8.341323) (end 9.005323 -8.341323) (width 0.25) (layer "F.Cu") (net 4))
 (segment (start 19.812 -12.908) (end 19.812 -9.652) (width 0.25) (layer "F.Cu") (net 4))
 (segment (start 1.456 -7.13175) (end 0.508 -8.07975) (width 0.25) (layer "F.Cu") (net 4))
 (segment (start 10.6445 -9.8755) (end 10.6445 -8.341323) (width 0.25) (layer "F.Cu") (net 4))
 (segment (start 9.8945 -5.07225) (end 9.8945 -4.57975) (width 0.25) (layer "F.Cu") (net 4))
 (segment (start 8.284 -7.62) (end 8.284 -6.68275) (width 0.25) (layer "F.Cu") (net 4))
 (segment (start 17.620497 -15.099503) (end 19.812 -12.908) (width 0.25) (layer "F.Cu") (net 4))
 (segment (start 9.005323 -8.341323) (end 8.284 -7.62) (width 0.25) (layer "F.Cu") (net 4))
 (segment (start 10.57 -9.95) (end 10.6445 -9.8755) (width 0.25) (layer "F.Cu") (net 4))
 (segment (start 9.744501 -4.429751) (end 9.744501 -3.825499) (width 0.25) (layer "F.Cu") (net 4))
 (segment (start 8.284 -6.68275) (end 9.8945 -5.07225) (width 0.25) (layer "F.Cu") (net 4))
 (segment (start 9.8945 -4.57975) (end 9.744501 -4.429751) (width 0.25) (layer "F.Cu") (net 4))
 (segment (start 2.42 -15.099503) (end 17.620497 -15.099503) (width 0.25) (layer "F.Cu") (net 4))
 (via (at 16.615 -10.182) (size 0.6) (drill 0.4) (layers "F.Cu" "B.Cu") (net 4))
 (via (at 10.57 -9.95) (size 0.6) (drill 0.4) (layers "F.Cu" "B.Cu") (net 4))
 (via (at 18.034 -10.16) (size 0.6) (drill 0.4) (layers "F.Cu" "B.Cu") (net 4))
 (via (at 10.57 -15.05) (size 0.6) (drill 0.4) (layers "F.Cu" "B.Cu") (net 4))
 (segment (start 16.615 -10.182) (end 18.012 -10.182) (width 0.25) (layer "B.Cu") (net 4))
 (segment (start 18.012 -10.182) (end 18.034 -10.16) (width 0.25) (layer "B.Cu") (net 4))
 (segment (start 10.57 -15.05) (end 10.57 -9.95) (width 0.25) (layer "B.Cu") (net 4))
 (segment (start 2.505 -10) (end 2.505 -10.597577) (width 0.4) (layer "F.Cu") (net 1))
 (segment (start 4.895 -3.275) (end 4.895 -6.083396) (width 0.4) (layer "F.Cu") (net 1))
 (segment (start 9.34 -10.433396) (end 8.098606 -9.192002) (width 0.4) (layer "F.Cu") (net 1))
 (segment (start 9.34 -10.67) (end 9.34 -10.433396) (width 0.4) (layer "F.Cu") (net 1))
 (segment (start 8.62 -11.81) (end 8.055 -12.375) (width 0.4) (layer "F.Cu") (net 1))
 (segment (start 11.345 -2.925) (end 11.895 -2.925) (width 0.3) (layer "F.Cu") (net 1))
 (segment (start 3.845 -9.975) (end 4.42 -9.4) (width 0.4) (layer "F.Cu") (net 1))
 (segment (start 4.095 -3.125) (end 4.745 -3.125) (width 0.4) (layer "F.Cu") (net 1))
 (segment (start 8.055 -12.375) (end 2.9495 -12.375) (width 0.4) (layer "F.Cu") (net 1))
 (segment (start 11.3005 -5.343394) (end 11.3005 -6.9555) (width 0.3) (layer "F.Cu") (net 1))
 (segment (start 11.895 -2.925) (end 12.014501 -3.044501) (width 0.3) (layer "F.Cu") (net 1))
 (segment (start 11.37 -10.35) (end 11.37 -7.025) (width 0.4) (layer "F.Cu") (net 1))
 (segment (start 4.095 -2.05) (end 3.845 -1.8) (width 0.4) (layer "F.Cu") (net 1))
 (segment (start 4.895 -6.083396) (end 6.915802 -8.104198) (width 0.4) (layer "F.Cu") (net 1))
 (segment (start 8.003606 -9.192002) (end 6.915802 -8.104198) (width 0.4) (layer "F.Cu") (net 1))
 (segment (start 11.05 -10.67) (end 11.37 -10.35) (width 0.4) (layer "F.Cu") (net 1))
 (segment (start 2.9495 -12.375) (end 2.5745 -12) (width 0.4) (layer "F.Cu") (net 1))
 (segment (start 9.34 -10.67) (end 11.05 -10.67) (width 0.4) (layer "F.Cu") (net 1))
 (segment (start 4.095 -3.125) (end 4.095 -2.05) (width 0.4) (layer "F.Cu") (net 1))
 (segment (start 3.82 -9.975) (end 2.53 -9.975) (width 0.4) (layer "F.Cu") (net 1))
 (segment (start 4.745 -3.125) (end 4.895 -3.275) (width 0.4) (layer "F.Cu") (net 1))
 (segment (start 8.098606 -9.192002) (end 8.003606 -9.192002) (width 0.4) (layer "F.Cu") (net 1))
 (segment (start 8.676604 -11.81) (end 9.34 -11.146604) (width 0.4) (layer "F.Cu") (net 1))
 (segment (start 9.34 -11.146604) (end 9.34 -10.67) (width 0.4) (layer "F.Cu") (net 1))
 (segment (start 12.014501 -4.629393) (end 11.3005 -5.343394) (width 0.3) (layer "F.Cu") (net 1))
 (segment (start 12.014501 -3.044501) (end 12.014501 -4.629393) (width 0.3) (layer "F.Cu") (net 1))
 (via (at 2.505 -10.597577) (size 0.6) (drill 0.4) (layers "F.Cu" "B.Cu") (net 1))
 (via (at 2.5745 -12) (size 0.6) (drill 0.4) (layers "F.Cu" "B.Cu") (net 1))
 (via (at 4.42 -9.4) (size 0.6) (drill 0.4) (layers "F.Cu" "B.Cu") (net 1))
 (via (at 6.915802 -8.104198) (size 0.6) (drill 0.4) (layers "F.Cu" "B.Cu") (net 1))
 (segment (start 2.52 -11.9455) (end 2.5745 -12) (width 0.4) (layer "B.Cu") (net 1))
 (segment (start 5.62 -9.4) (end 6.915802 -8.104198) (width 0.4) (layer "B.Cu") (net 1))
 (segment (start 2.52 -10.619423) (end 2.52 -10.612577) (width 0.4) (layer "B.Cu") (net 1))
 (segment (start 2.52 -10.619423) (end 2.501577 -10.601) (width 0.4) (layer "B.Cu") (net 1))
 (segment (start 2.52 -10.612577) (end 2.505 -10.597577) (width 0.4) (layer "B.Cu") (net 1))
 (segment (start 4.42 -9.4) (end 5.62 -9.4) (width 0.4) (layer "B.Cu") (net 1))
 (segment (start 2.52 -10.619423) (end 2.52 -11.9455) (width 0.4) (layer "B.Cu") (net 1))
 (segment (start 6.291302 -8.221454) (end 6.291302 -8.362875) (width 0.25) (layer "F.Cu") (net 6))
 (segment (start 7.08 -9.151573) (end 7.08 -10.985) (width 0.25) (layer "F.Cu") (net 6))
 (segment (start 6.291302 -8.362875) (end 7.08 -9.151573) (width 0.25) (layer "F.Cu") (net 6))
 (segment (start 4.095 -5.075) (end 4.095 -6.025152) (width 0.25) (layer "F.Cu") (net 6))
 (segment (start 8.62 -10.79) (end 7.275 -10.79) (width 0.25) (layer "F.Cu") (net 6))
 (segment (start 4.095 -6.025152) (end 6.291302 -8.221454) (width 0.25) (layer "F.Cu") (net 6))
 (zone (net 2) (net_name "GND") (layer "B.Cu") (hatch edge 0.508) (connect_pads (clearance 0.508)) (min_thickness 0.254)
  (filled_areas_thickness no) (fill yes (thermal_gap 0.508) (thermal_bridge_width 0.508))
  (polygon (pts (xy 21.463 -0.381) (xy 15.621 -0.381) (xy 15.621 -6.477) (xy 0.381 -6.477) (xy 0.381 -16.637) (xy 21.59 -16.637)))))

